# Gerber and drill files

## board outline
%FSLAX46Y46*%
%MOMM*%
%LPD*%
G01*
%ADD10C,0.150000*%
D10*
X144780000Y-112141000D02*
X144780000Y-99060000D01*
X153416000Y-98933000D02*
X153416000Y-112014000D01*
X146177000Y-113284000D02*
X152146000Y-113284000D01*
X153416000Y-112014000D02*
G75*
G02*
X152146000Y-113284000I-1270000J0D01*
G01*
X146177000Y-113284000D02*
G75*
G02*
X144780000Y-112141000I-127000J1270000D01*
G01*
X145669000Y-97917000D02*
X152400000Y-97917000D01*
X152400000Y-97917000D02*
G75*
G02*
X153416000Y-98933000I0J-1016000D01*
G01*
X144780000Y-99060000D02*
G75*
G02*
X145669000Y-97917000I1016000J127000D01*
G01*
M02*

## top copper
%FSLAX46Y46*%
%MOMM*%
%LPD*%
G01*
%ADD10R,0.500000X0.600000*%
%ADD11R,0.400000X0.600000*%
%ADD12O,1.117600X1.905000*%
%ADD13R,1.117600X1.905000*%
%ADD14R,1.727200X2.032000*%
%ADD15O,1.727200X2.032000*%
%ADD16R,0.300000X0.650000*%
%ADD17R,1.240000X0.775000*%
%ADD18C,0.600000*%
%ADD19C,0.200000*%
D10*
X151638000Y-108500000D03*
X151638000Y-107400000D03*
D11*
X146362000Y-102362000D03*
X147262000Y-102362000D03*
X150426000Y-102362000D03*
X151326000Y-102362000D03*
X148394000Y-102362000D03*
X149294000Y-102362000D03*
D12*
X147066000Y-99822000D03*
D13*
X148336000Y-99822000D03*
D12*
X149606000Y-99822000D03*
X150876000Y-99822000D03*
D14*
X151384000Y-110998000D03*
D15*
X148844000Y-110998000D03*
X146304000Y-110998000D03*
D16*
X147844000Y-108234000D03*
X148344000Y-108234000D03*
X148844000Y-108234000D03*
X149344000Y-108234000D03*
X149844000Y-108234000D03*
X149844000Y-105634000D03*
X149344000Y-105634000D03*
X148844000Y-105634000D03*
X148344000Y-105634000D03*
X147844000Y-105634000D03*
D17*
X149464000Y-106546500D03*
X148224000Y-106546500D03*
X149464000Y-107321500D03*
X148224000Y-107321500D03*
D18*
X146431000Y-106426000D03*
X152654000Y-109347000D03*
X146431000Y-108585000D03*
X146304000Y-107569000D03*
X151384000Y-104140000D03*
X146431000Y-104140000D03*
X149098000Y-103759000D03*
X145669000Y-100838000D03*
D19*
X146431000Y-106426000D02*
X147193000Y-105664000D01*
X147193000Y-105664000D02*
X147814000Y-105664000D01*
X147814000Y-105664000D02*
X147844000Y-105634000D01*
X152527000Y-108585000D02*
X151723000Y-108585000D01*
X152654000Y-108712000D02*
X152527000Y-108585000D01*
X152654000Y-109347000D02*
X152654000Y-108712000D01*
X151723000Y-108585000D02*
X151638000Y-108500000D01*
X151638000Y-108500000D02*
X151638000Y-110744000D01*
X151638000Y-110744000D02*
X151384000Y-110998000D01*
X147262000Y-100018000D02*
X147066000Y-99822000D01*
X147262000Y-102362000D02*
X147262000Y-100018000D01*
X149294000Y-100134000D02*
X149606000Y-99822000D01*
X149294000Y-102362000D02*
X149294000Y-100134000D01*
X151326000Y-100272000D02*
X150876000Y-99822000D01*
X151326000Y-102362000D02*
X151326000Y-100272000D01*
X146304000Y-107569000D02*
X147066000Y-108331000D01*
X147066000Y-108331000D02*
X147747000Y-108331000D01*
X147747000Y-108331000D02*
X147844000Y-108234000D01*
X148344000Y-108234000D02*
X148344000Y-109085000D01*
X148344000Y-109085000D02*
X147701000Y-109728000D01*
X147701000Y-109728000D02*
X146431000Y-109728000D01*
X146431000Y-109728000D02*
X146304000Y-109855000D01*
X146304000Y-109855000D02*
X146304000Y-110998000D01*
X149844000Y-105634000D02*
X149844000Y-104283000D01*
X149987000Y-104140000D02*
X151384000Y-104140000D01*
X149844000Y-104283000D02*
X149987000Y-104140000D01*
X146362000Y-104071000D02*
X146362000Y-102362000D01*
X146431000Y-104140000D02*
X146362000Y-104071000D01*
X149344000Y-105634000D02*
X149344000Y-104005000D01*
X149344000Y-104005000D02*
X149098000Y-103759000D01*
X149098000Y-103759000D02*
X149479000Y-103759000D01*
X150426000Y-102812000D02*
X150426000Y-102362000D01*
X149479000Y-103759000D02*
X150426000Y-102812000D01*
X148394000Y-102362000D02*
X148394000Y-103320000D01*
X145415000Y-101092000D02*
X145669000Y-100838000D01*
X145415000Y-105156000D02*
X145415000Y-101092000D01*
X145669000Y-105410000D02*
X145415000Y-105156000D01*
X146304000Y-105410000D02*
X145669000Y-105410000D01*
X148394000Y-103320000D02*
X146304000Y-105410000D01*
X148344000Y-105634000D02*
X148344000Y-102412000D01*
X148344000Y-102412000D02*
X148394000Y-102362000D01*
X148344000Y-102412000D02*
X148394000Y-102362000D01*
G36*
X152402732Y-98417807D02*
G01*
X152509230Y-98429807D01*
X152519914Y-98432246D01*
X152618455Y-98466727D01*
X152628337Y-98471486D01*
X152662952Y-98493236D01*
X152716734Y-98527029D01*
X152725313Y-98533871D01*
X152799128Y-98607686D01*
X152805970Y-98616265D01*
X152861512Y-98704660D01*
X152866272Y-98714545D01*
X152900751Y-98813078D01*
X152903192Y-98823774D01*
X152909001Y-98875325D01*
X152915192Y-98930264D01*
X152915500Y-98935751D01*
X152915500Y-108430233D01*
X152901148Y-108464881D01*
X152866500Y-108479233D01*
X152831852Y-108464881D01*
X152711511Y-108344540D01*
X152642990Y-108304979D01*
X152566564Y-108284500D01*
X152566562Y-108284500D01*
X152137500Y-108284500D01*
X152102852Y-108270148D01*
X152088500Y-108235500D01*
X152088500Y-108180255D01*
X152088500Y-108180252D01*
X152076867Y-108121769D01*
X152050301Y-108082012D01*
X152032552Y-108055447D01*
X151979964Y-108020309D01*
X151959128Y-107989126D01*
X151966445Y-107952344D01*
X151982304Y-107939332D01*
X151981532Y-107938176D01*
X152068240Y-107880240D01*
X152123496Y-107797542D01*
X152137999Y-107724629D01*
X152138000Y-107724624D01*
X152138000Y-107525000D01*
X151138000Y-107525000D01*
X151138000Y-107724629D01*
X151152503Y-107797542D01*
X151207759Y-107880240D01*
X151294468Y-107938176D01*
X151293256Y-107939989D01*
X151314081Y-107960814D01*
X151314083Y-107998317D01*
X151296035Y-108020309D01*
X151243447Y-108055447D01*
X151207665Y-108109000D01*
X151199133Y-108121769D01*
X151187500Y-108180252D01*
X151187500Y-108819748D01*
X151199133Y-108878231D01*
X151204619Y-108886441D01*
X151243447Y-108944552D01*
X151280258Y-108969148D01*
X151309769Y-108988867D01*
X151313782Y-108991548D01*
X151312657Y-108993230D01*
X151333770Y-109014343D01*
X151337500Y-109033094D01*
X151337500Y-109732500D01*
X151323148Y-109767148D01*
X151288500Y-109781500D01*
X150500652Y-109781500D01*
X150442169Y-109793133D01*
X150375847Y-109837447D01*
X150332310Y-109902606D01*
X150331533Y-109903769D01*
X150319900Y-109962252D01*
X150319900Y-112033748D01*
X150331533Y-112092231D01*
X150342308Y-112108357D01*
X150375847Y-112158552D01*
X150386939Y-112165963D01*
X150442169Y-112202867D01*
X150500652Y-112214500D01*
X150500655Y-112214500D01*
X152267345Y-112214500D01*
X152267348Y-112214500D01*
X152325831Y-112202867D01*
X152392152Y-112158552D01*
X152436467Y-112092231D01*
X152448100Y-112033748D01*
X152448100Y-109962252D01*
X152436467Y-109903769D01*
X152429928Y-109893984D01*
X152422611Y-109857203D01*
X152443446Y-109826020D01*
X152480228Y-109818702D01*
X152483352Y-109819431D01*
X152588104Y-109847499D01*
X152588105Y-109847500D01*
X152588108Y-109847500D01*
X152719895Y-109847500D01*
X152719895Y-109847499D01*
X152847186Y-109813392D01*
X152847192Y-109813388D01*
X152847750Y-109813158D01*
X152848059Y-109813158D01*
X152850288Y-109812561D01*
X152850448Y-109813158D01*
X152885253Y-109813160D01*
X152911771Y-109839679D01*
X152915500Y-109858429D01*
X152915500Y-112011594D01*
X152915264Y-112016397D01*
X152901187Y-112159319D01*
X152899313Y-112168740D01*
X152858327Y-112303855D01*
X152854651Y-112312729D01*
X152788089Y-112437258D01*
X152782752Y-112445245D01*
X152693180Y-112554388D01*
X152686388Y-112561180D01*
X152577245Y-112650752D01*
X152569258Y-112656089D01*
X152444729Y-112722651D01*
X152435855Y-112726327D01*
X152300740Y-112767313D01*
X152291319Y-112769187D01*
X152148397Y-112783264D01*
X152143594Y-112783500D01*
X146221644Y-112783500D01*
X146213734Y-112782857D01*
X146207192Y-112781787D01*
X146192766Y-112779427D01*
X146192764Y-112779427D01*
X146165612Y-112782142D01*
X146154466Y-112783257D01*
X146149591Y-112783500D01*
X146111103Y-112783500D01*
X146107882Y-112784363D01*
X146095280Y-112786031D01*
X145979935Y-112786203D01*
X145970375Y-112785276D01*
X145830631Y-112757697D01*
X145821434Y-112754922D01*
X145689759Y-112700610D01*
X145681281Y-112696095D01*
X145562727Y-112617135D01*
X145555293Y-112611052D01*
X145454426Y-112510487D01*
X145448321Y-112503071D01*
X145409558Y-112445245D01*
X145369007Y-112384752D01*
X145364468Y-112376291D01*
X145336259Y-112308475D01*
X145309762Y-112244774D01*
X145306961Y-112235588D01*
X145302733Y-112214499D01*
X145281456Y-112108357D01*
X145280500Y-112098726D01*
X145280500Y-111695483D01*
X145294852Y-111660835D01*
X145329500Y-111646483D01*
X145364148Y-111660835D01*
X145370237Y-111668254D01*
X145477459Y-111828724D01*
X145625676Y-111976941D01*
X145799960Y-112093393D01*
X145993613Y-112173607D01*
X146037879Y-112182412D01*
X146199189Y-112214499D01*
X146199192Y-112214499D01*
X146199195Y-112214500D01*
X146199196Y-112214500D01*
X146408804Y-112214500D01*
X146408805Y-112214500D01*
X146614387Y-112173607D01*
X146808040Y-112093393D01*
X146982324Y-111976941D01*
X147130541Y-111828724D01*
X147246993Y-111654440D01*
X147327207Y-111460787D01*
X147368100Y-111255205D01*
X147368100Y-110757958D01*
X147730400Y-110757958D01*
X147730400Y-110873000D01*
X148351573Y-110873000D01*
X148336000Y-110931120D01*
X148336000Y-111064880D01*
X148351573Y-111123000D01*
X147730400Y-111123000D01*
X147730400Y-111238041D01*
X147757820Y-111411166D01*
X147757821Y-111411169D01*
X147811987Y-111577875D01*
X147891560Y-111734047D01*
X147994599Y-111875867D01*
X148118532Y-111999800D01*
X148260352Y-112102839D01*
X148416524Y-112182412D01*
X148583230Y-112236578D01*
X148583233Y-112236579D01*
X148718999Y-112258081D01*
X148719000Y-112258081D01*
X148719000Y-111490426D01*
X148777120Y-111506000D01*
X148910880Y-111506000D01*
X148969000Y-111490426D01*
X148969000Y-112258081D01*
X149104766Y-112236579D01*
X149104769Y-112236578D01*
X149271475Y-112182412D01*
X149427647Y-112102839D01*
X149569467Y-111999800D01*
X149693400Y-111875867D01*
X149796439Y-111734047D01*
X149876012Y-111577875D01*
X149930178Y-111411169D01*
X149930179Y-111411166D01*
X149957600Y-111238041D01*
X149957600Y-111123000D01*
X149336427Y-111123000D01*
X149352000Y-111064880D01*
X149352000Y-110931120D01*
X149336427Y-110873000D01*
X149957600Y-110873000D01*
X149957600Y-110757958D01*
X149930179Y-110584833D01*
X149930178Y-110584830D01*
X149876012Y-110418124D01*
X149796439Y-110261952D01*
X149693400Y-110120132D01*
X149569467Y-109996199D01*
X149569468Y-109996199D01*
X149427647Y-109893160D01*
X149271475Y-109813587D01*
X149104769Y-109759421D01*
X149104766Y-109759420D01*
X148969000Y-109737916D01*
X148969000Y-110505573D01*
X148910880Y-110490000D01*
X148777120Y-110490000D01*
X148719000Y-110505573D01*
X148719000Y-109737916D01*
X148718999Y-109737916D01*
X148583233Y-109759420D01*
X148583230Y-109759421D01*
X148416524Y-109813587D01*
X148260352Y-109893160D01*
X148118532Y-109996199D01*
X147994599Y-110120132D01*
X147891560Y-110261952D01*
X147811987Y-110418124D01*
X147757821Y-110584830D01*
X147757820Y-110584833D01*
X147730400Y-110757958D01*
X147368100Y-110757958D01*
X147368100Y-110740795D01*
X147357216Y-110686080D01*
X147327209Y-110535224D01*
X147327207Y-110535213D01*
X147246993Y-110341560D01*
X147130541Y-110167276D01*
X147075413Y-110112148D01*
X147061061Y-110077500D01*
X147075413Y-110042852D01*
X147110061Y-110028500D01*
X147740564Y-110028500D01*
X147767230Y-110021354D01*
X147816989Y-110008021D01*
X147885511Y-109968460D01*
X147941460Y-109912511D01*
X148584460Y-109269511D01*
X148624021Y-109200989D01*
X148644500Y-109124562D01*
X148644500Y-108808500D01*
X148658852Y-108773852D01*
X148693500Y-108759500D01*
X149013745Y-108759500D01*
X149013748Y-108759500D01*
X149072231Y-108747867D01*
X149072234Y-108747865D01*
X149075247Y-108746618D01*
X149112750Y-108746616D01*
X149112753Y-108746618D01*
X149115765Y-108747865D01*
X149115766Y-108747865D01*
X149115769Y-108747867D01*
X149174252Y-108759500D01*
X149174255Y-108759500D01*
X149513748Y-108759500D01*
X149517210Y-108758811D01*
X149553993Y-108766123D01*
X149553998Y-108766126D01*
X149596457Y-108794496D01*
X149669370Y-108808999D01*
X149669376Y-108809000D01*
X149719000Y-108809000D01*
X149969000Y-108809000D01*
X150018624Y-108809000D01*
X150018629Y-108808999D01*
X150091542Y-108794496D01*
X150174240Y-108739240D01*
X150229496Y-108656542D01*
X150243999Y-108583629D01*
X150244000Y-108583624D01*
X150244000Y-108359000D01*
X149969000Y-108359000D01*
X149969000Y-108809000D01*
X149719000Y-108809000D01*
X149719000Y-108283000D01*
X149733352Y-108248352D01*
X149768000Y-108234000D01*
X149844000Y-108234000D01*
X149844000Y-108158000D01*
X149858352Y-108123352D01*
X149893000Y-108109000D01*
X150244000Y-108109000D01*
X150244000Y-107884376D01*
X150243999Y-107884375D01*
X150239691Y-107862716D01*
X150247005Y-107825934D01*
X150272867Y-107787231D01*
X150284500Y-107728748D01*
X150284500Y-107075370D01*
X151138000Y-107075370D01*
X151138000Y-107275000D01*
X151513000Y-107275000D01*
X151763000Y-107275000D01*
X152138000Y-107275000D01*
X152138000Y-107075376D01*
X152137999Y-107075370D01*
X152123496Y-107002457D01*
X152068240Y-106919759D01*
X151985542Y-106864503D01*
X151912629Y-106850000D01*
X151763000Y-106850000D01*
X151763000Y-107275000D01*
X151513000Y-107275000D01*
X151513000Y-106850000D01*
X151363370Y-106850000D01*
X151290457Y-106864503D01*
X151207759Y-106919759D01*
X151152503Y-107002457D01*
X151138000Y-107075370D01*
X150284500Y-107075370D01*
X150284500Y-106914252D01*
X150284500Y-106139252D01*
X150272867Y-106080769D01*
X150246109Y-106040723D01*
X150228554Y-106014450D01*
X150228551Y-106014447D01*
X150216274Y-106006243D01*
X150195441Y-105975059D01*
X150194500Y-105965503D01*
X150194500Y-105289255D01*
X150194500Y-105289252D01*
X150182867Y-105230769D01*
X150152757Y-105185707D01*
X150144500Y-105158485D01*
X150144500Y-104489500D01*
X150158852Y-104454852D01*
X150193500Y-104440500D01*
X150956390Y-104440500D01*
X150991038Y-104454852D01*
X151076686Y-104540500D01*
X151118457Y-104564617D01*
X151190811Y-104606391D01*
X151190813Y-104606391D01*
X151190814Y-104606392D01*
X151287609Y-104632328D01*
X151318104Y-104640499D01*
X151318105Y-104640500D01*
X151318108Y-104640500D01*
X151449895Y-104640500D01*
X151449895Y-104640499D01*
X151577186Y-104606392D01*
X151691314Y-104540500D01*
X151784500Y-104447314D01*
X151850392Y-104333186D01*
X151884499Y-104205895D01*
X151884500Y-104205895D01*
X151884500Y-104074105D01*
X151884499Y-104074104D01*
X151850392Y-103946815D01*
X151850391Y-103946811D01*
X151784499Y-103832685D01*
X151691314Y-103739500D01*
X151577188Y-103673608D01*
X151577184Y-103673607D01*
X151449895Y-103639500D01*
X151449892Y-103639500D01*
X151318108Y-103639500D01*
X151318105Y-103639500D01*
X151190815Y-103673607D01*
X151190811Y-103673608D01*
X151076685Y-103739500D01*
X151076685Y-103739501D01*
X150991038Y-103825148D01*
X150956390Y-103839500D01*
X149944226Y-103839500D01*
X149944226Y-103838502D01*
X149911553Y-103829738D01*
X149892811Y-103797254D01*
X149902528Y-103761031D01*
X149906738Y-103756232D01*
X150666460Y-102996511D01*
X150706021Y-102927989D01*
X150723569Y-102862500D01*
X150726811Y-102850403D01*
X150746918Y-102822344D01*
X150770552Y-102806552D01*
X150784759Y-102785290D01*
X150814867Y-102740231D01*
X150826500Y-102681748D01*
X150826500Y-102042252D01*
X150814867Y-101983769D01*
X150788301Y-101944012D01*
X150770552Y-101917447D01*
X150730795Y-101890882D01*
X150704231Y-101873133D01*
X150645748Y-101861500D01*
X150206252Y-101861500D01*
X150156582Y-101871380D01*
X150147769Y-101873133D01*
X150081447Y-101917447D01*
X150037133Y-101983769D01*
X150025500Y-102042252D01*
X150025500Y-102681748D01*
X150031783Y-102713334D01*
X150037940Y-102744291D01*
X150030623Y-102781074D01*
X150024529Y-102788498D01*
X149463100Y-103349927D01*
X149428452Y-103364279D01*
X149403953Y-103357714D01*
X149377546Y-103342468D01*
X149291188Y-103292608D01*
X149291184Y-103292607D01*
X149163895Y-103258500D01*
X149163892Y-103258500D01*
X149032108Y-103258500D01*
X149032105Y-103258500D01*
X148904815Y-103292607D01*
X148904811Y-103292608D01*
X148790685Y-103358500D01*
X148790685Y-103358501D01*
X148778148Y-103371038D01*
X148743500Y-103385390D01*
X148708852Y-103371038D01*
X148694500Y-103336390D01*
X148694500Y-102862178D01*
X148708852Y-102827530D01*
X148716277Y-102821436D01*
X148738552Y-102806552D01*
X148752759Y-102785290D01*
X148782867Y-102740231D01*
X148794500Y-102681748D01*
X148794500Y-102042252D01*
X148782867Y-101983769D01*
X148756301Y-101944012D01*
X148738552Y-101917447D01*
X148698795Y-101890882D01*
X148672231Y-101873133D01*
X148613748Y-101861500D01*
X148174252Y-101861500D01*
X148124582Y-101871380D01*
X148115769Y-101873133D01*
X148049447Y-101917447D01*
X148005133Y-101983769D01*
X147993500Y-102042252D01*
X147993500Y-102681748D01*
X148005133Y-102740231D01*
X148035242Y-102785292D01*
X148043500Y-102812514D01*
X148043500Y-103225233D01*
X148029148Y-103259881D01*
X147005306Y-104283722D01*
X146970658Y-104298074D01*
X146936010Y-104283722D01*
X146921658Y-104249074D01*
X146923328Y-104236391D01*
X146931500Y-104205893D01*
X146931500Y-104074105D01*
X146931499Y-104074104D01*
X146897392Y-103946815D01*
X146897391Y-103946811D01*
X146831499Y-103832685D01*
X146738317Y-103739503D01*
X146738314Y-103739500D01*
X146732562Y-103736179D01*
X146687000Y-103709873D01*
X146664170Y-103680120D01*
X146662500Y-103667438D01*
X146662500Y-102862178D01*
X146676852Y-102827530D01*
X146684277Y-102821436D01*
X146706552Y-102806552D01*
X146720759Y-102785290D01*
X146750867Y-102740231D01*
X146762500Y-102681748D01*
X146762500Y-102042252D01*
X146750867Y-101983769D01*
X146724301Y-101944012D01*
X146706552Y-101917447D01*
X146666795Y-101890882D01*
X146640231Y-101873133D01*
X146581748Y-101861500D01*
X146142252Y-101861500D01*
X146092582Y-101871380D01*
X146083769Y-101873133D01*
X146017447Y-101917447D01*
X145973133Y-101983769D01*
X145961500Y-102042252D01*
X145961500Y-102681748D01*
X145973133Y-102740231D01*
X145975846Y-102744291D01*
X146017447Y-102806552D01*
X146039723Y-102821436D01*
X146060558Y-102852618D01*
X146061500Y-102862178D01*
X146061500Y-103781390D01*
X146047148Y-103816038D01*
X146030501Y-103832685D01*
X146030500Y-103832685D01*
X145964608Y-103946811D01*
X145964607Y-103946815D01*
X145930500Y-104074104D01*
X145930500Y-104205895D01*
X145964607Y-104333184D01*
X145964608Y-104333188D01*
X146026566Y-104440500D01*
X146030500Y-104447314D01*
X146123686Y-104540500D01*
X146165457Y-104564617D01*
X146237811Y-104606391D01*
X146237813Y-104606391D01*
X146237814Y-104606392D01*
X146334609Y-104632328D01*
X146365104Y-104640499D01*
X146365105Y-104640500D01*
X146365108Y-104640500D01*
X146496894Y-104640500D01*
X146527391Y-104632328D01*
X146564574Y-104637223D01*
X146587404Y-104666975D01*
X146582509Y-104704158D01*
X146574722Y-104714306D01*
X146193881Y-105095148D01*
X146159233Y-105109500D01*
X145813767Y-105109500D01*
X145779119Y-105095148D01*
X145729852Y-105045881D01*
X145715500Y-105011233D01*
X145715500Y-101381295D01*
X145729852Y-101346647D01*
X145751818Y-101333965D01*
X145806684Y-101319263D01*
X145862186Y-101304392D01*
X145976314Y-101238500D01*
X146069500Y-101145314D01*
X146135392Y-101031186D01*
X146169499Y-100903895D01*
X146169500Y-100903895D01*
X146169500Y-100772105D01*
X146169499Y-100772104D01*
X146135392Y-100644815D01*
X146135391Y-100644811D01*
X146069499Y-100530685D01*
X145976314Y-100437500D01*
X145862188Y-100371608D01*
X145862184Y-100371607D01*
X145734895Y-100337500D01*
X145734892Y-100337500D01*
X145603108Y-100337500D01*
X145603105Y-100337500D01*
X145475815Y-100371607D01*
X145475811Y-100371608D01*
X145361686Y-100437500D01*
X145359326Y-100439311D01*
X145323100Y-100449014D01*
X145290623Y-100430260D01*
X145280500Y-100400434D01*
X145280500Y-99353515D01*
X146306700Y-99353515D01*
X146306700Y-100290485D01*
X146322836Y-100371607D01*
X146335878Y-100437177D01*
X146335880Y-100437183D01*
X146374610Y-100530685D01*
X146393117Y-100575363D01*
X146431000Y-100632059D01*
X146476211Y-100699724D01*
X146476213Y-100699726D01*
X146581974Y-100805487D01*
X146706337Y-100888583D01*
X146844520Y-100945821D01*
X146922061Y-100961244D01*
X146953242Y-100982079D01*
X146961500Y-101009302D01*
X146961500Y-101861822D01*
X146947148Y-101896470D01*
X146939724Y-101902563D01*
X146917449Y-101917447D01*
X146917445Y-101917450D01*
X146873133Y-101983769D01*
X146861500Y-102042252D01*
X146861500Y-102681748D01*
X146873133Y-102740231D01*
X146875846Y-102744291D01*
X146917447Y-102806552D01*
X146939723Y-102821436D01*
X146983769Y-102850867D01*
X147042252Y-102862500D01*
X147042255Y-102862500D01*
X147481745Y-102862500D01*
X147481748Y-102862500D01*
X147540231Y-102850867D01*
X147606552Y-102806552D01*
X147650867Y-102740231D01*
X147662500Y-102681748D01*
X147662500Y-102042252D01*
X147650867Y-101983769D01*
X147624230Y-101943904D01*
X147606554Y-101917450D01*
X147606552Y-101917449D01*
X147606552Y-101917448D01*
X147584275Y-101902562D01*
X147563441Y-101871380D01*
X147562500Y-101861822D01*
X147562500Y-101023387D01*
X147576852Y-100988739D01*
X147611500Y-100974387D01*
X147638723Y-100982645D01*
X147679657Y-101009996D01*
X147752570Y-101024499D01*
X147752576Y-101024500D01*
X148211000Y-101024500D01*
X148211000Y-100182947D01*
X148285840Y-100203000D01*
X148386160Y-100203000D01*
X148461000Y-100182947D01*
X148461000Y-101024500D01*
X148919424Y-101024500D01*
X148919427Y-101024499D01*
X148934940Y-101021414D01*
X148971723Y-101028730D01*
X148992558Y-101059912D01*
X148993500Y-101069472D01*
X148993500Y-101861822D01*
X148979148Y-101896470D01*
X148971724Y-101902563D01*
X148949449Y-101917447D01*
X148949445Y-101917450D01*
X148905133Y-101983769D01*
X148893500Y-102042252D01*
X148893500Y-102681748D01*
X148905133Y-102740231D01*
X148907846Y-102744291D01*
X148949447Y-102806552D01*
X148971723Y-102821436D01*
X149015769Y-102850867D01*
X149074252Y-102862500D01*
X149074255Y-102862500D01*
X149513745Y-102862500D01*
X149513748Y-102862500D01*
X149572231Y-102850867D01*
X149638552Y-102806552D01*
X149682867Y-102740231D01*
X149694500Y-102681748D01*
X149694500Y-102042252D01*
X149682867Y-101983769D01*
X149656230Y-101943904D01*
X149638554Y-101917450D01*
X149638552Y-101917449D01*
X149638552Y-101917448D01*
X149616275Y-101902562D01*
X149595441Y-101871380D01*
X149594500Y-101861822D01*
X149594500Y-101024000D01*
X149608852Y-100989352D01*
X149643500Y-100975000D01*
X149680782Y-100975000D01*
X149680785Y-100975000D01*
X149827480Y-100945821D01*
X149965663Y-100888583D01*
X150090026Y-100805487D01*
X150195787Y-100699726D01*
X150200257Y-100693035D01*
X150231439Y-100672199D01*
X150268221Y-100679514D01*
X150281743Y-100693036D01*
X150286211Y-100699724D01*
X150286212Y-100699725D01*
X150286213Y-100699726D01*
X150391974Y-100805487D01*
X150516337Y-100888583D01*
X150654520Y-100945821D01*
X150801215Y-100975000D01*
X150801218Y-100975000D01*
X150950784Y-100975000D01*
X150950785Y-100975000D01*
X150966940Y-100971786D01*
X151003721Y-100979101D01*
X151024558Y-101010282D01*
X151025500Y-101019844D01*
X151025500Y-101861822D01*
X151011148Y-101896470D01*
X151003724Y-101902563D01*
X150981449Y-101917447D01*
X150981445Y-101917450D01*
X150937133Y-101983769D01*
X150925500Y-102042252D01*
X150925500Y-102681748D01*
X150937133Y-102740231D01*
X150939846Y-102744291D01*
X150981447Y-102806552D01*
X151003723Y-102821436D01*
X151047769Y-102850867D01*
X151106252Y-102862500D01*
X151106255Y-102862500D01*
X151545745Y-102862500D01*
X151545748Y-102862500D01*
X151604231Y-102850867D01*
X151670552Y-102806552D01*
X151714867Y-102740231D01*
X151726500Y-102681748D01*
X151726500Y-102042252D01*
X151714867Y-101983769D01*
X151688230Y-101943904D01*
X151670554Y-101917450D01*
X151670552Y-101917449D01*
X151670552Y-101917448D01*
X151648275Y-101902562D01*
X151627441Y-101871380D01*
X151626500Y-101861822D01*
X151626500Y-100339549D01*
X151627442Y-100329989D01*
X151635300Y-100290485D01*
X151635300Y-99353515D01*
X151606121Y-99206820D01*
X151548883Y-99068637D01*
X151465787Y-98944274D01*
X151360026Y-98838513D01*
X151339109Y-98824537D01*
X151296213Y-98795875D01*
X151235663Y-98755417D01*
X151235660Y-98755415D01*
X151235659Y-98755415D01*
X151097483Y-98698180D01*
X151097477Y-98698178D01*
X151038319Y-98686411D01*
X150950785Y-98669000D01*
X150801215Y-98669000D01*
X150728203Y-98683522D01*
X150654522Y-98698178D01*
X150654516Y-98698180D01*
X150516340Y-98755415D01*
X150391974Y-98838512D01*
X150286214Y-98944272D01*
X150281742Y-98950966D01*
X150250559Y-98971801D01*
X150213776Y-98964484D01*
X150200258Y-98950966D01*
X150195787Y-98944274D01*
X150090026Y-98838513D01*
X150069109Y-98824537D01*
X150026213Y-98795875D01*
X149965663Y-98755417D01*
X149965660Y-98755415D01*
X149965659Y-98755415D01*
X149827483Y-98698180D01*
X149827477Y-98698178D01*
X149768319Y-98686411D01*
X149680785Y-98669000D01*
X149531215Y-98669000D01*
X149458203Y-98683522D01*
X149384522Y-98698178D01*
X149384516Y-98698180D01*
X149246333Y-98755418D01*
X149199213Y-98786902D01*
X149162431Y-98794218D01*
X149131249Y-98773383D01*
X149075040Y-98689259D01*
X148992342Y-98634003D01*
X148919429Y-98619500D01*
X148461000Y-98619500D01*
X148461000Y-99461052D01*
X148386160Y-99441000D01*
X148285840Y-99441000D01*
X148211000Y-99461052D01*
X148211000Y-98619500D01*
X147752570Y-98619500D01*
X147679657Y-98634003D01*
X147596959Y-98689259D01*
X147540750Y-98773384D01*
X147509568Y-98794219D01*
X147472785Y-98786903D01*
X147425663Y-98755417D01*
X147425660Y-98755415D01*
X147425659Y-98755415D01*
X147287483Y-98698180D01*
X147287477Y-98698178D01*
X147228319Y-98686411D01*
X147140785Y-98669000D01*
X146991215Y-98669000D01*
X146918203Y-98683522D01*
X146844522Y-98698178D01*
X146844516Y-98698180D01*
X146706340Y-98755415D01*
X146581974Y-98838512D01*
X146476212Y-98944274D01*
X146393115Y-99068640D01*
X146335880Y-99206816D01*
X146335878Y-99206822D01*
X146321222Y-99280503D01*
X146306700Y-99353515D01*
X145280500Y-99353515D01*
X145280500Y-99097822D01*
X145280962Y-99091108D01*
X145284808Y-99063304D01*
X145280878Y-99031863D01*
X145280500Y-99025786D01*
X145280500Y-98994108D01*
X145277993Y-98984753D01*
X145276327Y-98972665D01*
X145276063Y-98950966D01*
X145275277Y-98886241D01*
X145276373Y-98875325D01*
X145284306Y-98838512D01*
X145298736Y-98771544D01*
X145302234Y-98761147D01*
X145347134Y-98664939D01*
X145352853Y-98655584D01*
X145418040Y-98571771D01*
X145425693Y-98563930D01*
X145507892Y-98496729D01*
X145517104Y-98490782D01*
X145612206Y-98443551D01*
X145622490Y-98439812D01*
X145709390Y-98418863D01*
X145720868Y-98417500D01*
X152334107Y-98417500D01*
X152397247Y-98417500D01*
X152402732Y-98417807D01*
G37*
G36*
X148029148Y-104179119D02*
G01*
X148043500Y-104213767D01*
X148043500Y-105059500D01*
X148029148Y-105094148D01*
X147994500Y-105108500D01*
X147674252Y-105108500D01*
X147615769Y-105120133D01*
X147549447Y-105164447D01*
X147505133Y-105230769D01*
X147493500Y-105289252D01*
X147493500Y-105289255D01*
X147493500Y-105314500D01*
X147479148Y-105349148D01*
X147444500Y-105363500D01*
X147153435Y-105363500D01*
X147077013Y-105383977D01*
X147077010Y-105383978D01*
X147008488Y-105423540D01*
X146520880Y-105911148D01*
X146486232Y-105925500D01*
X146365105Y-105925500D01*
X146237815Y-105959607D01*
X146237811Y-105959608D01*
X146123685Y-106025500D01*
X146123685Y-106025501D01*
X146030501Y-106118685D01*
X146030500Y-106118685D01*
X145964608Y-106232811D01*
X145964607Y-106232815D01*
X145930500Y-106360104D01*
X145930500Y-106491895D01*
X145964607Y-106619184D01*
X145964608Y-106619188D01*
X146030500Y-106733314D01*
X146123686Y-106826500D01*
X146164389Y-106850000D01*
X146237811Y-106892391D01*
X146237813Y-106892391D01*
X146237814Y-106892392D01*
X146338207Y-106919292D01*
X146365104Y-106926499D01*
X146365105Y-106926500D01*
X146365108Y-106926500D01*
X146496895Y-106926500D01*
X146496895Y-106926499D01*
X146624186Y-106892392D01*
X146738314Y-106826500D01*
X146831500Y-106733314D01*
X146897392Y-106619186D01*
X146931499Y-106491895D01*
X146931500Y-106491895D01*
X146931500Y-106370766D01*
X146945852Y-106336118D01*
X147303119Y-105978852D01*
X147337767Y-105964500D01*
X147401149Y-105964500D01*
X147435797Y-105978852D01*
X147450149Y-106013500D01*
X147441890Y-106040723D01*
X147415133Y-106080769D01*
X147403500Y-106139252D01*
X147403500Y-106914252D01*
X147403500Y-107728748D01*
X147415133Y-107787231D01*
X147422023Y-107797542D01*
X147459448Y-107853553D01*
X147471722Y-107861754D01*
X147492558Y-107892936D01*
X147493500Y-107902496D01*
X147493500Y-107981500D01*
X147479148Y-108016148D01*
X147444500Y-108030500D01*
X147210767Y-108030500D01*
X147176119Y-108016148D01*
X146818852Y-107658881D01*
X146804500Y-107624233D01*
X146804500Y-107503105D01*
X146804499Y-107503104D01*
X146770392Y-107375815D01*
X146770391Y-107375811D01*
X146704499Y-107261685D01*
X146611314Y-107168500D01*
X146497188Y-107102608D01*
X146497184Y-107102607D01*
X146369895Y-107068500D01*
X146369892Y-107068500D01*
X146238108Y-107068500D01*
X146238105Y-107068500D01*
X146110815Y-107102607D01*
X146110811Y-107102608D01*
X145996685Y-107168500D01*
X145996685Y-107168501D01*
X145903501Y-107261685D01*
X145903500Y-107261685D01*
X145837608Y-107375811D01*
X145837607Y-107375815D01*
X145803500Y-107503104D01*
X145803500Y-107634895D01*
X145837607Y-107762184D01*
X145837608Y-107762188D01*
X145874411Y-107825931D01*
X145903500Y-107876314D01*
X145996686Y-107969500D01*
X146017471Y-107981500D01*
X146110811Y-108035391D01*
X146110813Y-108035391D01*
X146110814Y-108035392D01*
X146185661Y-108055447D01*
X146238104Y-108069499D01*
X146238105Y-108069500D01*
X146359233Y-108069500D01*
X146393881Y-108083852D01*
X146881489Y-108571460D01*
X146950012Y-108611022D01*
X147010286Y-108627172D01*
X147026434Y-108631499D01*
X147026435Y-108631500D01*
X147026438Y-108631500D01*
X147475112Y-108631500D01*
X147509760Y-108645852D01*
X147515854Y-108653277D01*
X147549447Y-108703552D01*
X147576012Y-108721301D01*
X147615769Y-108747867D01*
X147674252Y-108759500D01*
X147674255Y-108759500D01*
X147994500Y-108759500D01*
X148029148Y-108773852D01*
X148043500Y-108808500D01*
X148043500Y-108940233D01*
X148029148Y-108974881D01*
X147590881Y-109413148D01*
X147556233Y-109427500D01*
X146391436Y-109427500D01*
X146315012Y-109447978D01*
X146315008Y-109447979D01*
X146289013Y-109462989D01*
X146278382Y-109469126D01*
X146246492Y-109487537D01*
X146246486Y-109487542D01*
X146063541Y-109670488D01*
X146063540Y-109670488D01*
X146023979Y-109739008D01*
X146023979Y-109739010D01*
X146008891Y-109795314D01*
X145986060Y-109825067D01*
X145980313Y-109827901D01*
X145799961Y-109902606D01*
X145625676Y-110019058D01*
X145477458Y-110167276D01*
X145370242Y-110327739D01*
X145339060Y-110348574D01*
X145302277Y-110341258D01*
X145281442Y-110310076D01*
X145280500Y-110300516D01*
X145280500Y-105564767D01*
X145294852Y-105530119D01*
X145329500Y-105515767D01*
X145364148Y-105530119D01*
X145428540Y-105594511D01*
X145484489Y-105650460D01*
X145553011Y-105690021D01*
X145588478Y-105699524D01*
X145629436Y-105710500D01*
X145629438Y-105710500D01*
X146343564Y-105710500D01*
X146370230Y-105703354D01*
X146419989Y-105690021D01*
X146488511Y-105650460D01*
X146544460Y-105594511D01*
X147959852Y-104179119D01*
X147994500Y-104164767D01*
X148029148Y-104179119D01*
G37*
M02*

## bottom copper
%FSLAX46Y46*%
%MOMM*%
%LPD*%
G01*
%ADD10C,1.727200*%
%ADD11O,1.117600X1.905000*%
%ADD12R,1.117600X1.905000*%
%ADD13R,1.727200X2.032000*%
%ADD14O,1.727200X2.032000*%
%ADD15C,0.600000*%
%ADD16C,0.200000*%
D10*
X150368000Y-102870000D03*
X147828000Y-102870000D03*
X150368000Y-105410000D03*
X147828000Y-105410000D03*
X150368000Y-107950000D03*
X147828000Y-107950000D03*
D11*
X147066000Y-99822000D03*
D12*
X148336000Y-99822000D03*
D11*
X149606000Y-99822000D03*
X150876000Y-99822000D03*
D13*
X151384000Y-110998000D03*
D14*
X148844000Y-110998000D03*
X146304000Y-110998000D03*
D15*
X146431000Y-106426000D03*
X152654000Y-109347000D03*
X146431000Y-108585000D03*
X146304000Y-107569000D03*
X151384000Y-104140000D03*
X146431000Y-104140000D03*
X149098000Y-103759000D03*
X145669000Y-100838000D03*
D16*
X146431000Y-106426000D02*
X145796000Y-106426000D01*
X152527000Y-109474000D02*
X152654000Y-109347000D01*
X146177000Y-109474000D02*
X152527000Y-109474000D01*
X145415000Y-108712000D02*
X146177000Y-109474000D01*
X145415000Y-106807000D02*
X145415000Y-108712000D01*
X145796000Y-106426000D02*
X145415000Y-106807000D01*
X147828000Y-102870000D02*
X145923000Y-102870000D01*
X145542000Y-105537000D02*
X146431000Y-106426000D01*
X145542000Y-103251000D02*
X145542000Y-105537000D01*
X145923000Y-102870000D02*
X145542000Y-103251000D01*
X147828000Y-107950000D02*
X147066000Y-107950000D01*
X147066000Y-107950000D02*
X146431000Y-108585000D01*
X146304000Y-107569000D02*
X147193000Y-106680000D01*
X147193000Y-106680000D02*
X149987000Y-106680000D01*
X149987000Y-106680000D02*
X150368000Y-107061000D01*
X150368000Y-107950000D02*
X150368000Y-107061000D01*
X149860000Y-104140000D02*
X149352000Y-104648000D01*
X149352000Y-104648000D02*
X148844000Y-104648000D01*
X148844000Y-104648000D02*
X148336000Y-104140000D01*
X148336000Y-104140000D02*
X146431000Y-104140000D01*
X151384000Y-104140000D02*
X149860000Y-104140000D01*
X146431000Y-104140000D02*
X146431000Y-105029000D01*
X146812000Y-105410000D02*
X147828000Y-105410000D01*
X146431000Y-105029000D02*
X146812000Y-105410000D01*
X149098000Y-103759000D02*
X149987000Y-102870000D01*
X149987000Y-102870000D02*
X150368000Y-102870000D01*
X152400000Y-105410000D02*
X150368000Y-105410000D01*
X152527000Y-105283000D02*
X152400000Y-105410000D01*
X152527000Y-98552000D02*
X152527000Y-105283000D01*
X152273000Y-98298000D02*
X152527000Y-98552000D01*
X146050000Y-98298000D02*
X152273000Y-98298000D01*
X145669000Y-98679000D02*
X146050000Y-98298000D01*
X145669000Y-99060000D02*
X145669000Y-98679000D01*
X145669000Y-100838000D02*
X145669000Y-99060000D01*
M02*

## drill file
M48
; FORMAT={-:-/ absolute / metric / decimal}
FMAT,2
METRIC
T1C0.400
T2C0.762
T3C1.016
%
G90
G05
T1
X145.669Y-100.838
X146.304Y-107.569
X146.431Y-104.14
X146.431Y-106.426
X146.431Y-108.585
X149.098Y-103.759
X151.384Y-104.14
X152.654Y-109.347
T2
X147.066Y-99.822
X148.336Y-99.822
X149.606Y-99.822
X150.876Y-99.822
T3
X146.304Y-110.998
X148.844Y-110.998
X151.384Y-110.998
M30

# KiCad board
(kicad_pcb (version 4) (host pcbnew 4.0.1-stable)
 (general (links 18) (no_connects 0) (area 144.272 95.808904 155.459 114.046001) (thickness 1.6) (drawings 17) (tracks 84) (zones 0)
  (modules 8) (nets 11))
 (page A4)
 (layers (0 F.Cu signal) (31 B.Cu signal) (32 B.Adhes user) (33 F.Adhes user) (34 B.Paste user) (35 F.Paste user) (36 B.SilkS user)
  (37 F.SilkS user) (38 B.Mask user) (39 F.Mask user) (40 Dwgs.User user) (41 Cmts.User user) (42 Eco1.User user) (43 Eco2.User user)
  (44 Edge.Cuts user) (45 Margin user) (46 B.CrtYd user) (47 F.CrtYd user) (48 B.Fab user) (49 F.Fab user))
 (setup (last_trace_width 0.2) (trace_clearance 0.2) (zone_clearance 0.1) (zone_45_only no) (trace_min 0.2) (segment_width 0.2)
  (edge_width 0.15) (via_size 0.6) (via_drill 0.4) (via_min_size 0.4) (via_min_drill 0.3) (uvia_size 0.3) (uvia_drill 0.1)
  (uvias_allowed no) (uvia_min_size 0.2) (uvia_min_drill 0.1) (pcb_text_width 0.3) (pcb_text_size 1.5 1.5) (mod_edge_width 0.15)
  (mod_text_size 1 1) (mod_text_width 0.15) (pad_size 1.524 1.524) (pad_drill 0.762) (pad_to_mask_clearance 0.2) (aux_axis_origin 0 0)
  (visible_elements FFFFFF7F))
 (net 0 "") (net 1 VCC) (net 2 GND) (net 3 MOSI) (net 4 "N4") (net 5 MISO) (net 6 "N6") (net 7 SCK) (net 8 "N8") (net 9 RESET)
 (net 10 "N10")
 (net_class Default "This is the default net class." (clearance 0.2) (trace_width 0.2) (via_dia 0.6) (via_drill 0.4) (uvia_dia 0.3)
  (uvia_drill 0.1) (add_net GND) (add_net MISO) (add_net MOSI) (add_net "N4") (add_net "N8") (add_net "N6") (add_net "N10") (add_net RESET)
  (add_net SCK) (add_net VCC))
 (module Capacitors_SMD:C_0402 (layer F.Cu) (at 151.638 107.95 90)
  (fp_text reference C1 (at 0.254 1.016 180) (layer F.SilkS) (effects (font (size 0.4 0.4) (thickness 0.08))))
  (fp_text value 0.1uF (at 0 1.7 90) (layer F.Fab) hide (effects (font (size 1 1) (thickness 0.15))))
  (pad 1 smd rect (at -0.55 0 90) (size 0.6 0.5) (layers F.Cu F.Paste F.Mask) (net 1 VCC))
  (pad 2 smd rect (at 0.55 0 90) (size 0.6 0.5) (layers F.Cu F.Paste F.Mask) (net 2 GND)))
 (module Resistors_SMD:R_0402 (layer F.Cu) (at 146.812 102.362)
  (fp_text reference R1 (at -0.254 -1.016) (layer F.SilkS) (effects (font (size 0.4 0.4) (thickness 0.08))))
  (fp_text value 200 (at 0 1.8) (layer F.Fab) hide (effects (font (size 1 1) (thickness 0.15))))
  (pad 1 smd rect (at -0.45 0) (size 0.4 0.6) (layers F.Cu F.Paste F.Mask) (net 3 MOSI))
  (pad 2 smd rect (at 0.45 0) (size 0.4 0.6) (layers F.Cu F.Paste F.Mask) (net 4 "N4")))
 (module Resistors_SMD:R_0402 (layer F.Cu) (at 150.876 102.362)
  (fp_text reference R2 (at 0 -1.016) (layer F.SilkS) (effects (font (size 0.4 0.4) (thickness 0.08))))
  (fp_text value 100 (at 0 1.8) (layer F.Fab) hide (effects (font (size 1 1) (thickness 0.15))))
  (pad 1 smd rect (at -0.45 0) (size 0.4 0.6) (layers F.Cu F.Paste F.Mask) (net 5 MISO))
  (pad 2 smd rect (at 0.45 0) (size 0.4 0.6) (layers F.Cu F.Paste F.Mask) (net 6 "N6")))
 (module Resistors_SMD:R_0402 (layer F.Cu) (at 148.844 102.362)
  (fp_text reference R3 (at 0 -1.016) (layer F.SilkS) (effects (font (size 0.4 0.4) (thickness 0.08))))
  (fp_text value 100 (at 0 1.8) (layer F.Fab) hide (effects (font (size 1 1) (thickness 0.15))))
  (pad 1 smd rect (at -0.45 0) (size 0.4 0.6) (layers F.Cu F.Paste F.Mask) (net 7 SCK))
  (pad 2 smd rect (at 0.45 0) (size 0.4 0.6) (layers F.Cu F.Paste F.Mask) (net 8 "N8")))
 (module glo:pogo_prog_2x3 (layer B.Cu) (at 150.368 102.87 180)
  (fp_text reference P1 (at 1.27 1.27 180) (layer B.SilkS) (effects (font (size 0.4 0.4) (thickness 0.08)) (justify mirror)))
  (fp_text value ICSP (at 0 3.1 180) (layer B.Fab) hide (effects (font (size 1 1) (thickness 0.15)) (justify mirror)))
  (pad 1 smd circle (at 0 0 180) (size 1.7272 1.7272) (layers B.Cu B.Paste B.Mask) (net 5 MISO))
  (pad 2 smd circle (at 2.54 0 180) (size 1.7272 1.7272) (layers B.Cu B.Paste B.Mask) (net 1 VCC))
  (pad 3 smd circle (at 0 -2.54 180) (size 1.7272 1.7272) (layers B.Cu B.Paste B.Mask) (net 7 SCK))
  (pad 4 smd circle (at 2.54 -2.54 180) (size 1.7272 1.7272) (layers B.Cu B.Paste B.Mask) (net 3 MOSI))
  (pad 5 smd circle (at 0 -5.08 180) (size 1.7272 1.7272) (layers B.Cu B.Paste B.Mask) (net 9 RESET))
  (pad 6 smd circle (at 2.54 -5.08 180) (size 1.7272 1.7272) (layers B.Cu B.Paste B.Mask) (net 2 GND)))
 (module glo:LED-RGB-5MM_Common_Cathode (layer F.Cu) (at 147.066 99.822 90)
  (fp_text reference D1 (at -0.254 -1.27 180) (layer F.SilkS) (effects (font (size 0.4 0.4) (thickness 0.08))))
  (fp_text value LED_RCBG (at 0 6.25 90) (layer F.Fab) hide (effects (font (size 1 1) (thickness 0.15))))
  (pad 1 thru_hole oval (at 0 0 90) (size 1.905 1.1176) (drill 0.762) (layers *.Cu *.Mask F.SilkS) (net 4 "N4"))
  (pad 2 thru_hole rect (at 0 1.27 90) (size 1.905 1.1176) (drill 0.762) (layers *.Cu *.Mask F.SilkS) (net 2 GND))
  (pad 3 thru_hole oval (at 0 2.54 90) (size 1.905 1.1176) (drill 0.762) (layers *.Cu *.Mask F.SilkS) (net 8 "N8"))
  (pad 4 thru_hole oval (at 0 3.81 90) (size 1.905 1.1176) (drill 0.762) (layers *.Cu *.Mask F.SilkS) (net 6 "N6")))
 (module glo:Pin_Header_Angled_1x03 (layer F.Cu) (at 151.384 110.998 270)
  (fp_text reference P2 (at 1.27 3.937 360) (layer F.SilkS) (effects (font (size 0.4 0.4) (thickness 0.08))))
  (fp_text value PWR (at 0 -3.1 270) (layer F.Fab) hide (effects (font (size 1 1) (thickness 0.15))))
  (pad 1 thru_hole rect (at 0 0 270) (size 2.032 1.7272) (drill 1.016) (layers *.Cu *.Mask F.SilkS) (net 1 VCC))
  (pad 2 thru_hole oval (at 0 2.54 270) (size 2.032 1.7272) (drill 1.016) (layers *.Cu *.Mask F.SilkS) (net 2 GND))
  (pad 3 thru_hole oval (at 0 5.08 270) (size 2.032 1.7272) (drill 1.016) (layers *.Cu *.Mask F.SilkS) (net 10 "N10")))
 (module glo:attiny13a (layer F.Cu) (at 148.844 106.934 90)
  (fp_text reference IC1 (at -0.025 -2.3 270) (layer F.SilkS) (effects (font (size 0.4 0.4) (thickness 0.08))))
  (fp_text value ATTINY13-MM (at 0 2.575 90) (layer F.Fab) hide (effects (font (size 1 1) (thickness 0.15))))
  (pad 1 smd rect (at -1.3 -1 90) (size 0.65 0.3) (layers F.Cu F.Paste F.Mask) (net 9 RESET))
  (pad 2 smd rect (at -1.3 -0.5 90) (size 0.65 0.3) (layers F.Cu F.Paste F.Mask) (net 10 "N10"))
  (pad 3 smd rect (at -1.3 0 90) (size 0.65 0.3) (layers F.Cu F.Paste F.Mask))
  (pad 4 smd rect (at -1.3 0.5 90) (size 0.65 0.3) (layers F.Cu F.Paste F.Mask))
  (pad 5 smd rect (at -1.3 1 90) (size 0.65 0.3) (layers F.Cu F.Paste F.Mask) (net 2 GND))
  (pad 6 smd rect (at 1.3 1 90) (size 0.65 0.3) (layers F.Cu F.Paste F.Mask) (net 3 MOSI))
  (pad 7 smd rect (at 1.3 0.5 90) (size 0.65 0.3) (layers F.Cu F.Paste F.Mask) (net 5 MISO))
  (pad 8 smd rect (at 1.3 0 90) (size 0.65 0.3) (layers F.Cu F.Paste F.Mask))
  (pad 9 smd rect (at 1.3 -0.5 90) (size 0.65 0.3) (layers F.Cu F.Paste F.Mask) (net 7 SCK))
  (pad 10 smd rect (at 1.3 -1 90) (size 0.65 0.3) (layers F.Cu F.Paste F.Mask) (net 1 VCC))
  (pad "" smd rect (at 0.3875 0.62 90) (size 0.775 1.24) (layers F.Cu F.Paste F.Mask) (solder_paste_margin_ratio -0.2))
  (pad "" smd rect (at 0.3875 -0.62 90) (size 0.775 1.24) (layers F.Cu F.Paste F.Mask) (solder_paste_margin_ratio -0.2))
  (pad "" smd rect (at -0.3875 0.62 90) (size 0.775 1.24) (layers F.Cu F.Paste F.Mask) (solder_paste_margin_ratio -0.2))
  (pad "" smd rect (at -0.3875 -0.62 90) (size 0.775 1.24) (layers F.Cu F.Paste F.Mask) (solder_paste_margin_ratio -0.2)))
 (gr_line (start 144.78 112.141) (end 144.78 99.06) (angle 90) (layer Edge.Cuts) (width 0.15))
 (gr_line (start 153.416 98.933) (end 153.416 112.014) (angle 90) (layer Edge.Cuts) (width 0.15))
 (gr_line (start 146.177 113.284) (end 152.146 113.284) (angle 90) (layer Edge.Cuts) (width 0.15))
 (gr_arc (start 152.146 112.014) (end 153.416 112.014) (angle 90) (layer Edge.Cuts) (width 0.15))
 (gr_arc (start 146.05 112.014) (end 146.177 113.284) (angle 90) (layer Edge.Cuts) (width 0.15))
 (gr_line (start 145.669 97.917) (end 152.4 97.917) (angle 90) (layer Edge.Cuts) (width 0.15))
 (gr_arc (start 152.4 98.933) (end 152.4 97.917) (angle 90) (layer Edge.Cuts) (width 0.15))
 (gr_arc (start 145.796 98.933) (end 144.78 99.06) (angle 90) (layer Edge.Cuts) (width 0.15))
 (segment (start 146.431 106.426) (end 147.193 105.664) (width 0.2) (layer F.Cu) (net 1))
 (via (at 146.431 106.426) (size 0.6) (drill 0.4) (layers F.Cu B.Cu) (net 1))
 (segment (start 147.193 105.664) (end 147.814 105.664) (width 0.2) (layer F.Cu) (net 1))
 (segment (start 147.814 105.664) (end 147.844 105.634) (width 0.2) (layer F.Cu) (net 1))
 (segment (start 146.431 106.426) (end 145.796 106.426) (width 0.2) (layer B.Cu) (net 1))
 (segment (start 152.527 108.585) (end 151.723 108.585) (width 0.2) (layer F.Cu) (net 1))
 (segment (start 152.654 108.712) (end 152.527 108.585) (width 0.2) (layer F.Cu) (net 1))
 (segment (start 152.654 109.347) (end 152.654 108.712) (width 0.2) (layer F.Cu) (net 1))
 (via (at 152.654 109.347) (size 0.6) (drill 0.4) (layers F.Cu B.Cu) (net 1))
 (segment (start 152.527 109.474) (end 152.654 109.347) (width 0.2) (layer B.Cu) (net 1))
 (segment (start 146.177 109.474) (end 152.527 109.474) (width 0.2) (layer B.Cu) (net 1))
 (segment (start 145.415 108.712) (end 146.177 109.474) (width 0.2) (layer B.Cu) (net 1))
 (segment (start 145.415 106.807) (end 145.415 108.712) (width 0.2) (layer B.Cu) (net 1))
 (segment (start 145.796 106.426) (end 145.415 106.807) (width 0.2) (layer B.Cu) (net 1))
 (segment (start 151.723 108.585) (end 151.638 108.5) (width 0.2) (layer F.Cu) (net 1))
 (segment (start 147.828 102.87) (end 145.923 102.87) (width 0.2) (layer B.Cu) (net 1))
 (segment (start 145.542 105.537) (end 146.431 106.426) (width 0.2) (layer B.Cu) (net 1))
 (segment (start 145.542 103.251) (end 145.542 105.537) (width 0.2) (layer B.Cu) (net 1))
 (segment (start 145.923 102.87) (end 145.542 103.251) (width 0.2) (layer B.Cu) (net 1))
 (segment (start 151.638 108.5) (end 151.638 110.744) (width 0.2) (layer F.Cu) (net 1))
 (segment (start 151.638 110.744) (end 151.384 110.998) (width 0.2) (layer F.Cu) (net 1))
 (segment (start 147.828 107.95) (end 147.066 107.95) (width 0.2) (layer B.Cu) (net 2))
 (segment (start 147.066 107.95) (end 146.431 108.585) (width 0.2) (layer B.Cu) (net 2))
 (via (at 146.431 108.585) (size 0.6) (drill 0.4) (layers F.Cu B.Cu) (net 2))
 (segment (start 147.262 100.018) (end 147.066 99.822) (width 0.2) (layer F.Cu) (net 4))
 (segment (start 147.262 102.362) (end 147.262 100.018) (width 0.2) (layer F.Cu) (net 4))
 (segment (start 149.294 100.134) (end 149.606 99.822) (width 0.2) (layer F.Cu) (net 8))
 (segment (start 149.294 102.362) (end 149.294 100.134) (width 0.2) (layer F.Cu) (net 8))
 (segment (start 151.326 100.272) (end 150.876 99.822) (width 0.2) (layer F.Cu) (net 6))
 (segment (start 151.326 102.362) (end 151.326 100.272) (width 0.2) (layer F.Cu) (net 6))
 (segment (start 146.304 107.569) (end 147.066 108.331) (width 0.2) (layer F.Cu) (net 9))
 (via (at 146.304 107.569) (size 0.6) (drill 0.4) (layers F.Cu B.Cu) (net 9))
 (segment (start 146.304 107.569) (end 147.193 106.68) (width 0.2) (layer B.Cu) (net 9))
 (segment (start 147.193 106.68) (end 149.987 106.68) (width 0.2) (layer B.Cu) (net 9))
 (segment (start 149.987 106.68) (end 150.368 107.061) (width 0.2) (layer B.Cu) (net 9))
 (segment (start 150.368 107.95) (end 150.368 107.061) (width 0.2) (layer B.Cu) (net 9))
 (segment (start 147.066 108.331) (end 147.747 108.331) (width 0.2) (layer F.Cu) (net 9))
 (segment (start 147.747 108.331) (end 147.844 108.234) (width 0.2) (layer F.Cu) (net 9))
 (segment (start 148.344 108.234) (end 148.344 109.085) (width 0.2) (layer F.Cu) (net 10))
 (segment (start 148.344 109.085) (end 147.701 109.728) (width 0.2) (layer F.Cu) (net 10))
 (segment (start 147.701 109.728) (end 146.431 109.728) (width 0.2) (layer F.Cu) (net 10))
 (segment (start 146.431 109.728) (end 146.304 109.855) (width 0.2) (layer F.Cu) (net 10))
 (segment (start 146.304 109.855) (end 146.304 110.998) (width 0.2) (layer F.Cu) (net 10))
 (segment (start 149.844 105.634) (end 149.844 104.283) (width 0.2) (layer F.Cu) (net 3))
 (segment (start 149.86 104.14) (end 149.352 104.648) (width 0.2) (layer B.Cu) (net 3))
 (segment (start 149.352 104.648) (end 148.844 104.648) (width 0.2) (layer B.Cu) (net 3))
 (segment (start 148.844 104.648) (end 148.336 104.14) (width 0.2) (layer B.Cu) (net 3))
 (segment (start 148.336 104.14) (end 146.431 104.14) (width 0.2) (layer B.Cu) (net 3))
 (via (at 151.384 104.14) (size 0.6) (drill 0.4) (layers F.Cu B.Cu) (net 3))
 (segment (start 149.987 104.14) (end 151.384 104.14) (width 0.2) (layer F.Cu) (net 3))
 (segment (start 149.844 104.283) (end 149.987 104.14) (width 0.2) (layer F.Cu) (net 3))
 (segment (start 151.384 104.14) (end 149.86 104.14) (width 0.2) (layer B.Cu) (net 3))
 (segment (start 146.431 104.14) (end 146.431 105.029) (width 0.2) (layer B.Cu) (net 3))
 (segment (start 146.812 105.41) (end 147.828 105.41) (width 0.2) (layer B.Cu) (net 3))
 (segment (start 146.431 105.029) (end 146.812 105.41) (width 0.2) (layer B.Cu) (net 3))
 (segment (start 146.362 104.071) (end 146.362 102.362) (width 0.2) (layer F.Cu) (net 3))
 (segment (start 146.431 104.14) (end 146.362 104.071) (width 0.2) (layer F.Cu) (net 3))
 (via (at 146.431 104.14) (size 0.6) (drill 0.4) (layers F.Cu B.Cu) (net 3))
 (segment (start 149.344 105.634) (end 149.344 104.005) (width 0.2) (layer F.Cu) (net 5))
 (segment (start 149.344 104.005) (end 149.098 103.759) (width 0.2) (layer F.Cu) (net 5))
 (segment (start 149.098 103.759) (end 149.479 103.759) (width 0.2) (layer F.Cu) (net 5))
 (segment (start 150.426 102.812) (end 150.426 102.362) (width 0.2) (layer F.Cu) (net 5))
 (segment (start 149.479 103.759) (end 150.426 102.812) (width 0.2) (layer F.Cu) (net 5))
 (segment (start 149.098 103.759) (end 149.987 102.87) (width 0.2) (layer B.Cu) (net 5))
 (via (at 149.098 103.759) (size 0.6) (drill 0.4) (layers F.Cu B.Cu) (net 5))
 (segment (start 149.987 102.87) (end 150.368 102.87) (width 0.2) (layer B.Cu) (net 5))
 (segment (start 148.394 102.362) (end 148.394 103.32) (width 0.2) (layer F.Cu) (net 7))
 (segment (start 152.4 105.41) (end 150.368 105.41) (width 0.2) (layer B.Cu) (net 7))
 (segment (start 152.527 105.283) (end 152.4 105.41) (width 0.2) (layer B.Cu) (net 7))
 (segment (start 152.527 98.552) (end 152.527 105.283) (width 0.2) (layer B.Cu) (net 7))
 (segment (start 152.273 98.298) (end 152.527 98.552) (width 0.2) (layer B.Cu) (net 7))
 (segment (start 146.05 98.298) (end 152.273 98.298) (width 0.2) (layer B.Cu) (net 7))
 (segment (start 145.669 98.679) (end 146.05 98.298) (width 0.2) (layer B.Cu) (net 7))
 (segment (start 145.669 99.06) (end 145.669 98.679) (width 0.2) (layer B.Cu) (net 7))
 (segment (start 145.669 100.838) (end 145.669 99.06) (width 0.2) (layer B.Cu) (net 7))
 (via (at 145.669 100.838) (size 0.6) (drill 0.4) (layers F.Cu B.Cu) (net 7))
 (segment (start 145.415 101.092) (end 145.669 100.838) (width 0.2) (layer F.Cu) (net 7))
 (segment (start 145.415 105.156) (end 145.415 101.092) (width 0.2) (layer F.Cu) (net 7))
 (segment (start 145.669 105.41) (end 145.415 105.156) (width 0.2) (layer F.Cu) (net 7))
 (segment (start 146.304 105.41) (end 145.669 105.41) (width 0.2) (layer F.Cu) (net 7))
 (segment (start 148.394 103.32) (end 146.304 105.41) (width 0.2) (layer F.Cu) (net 7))
 (segment (start 148.344 105.634) (end 148.344 102.412) (width 0.2) (layer F.Cu) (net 7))
 (segment (start 148.344 102.412) (end 148.394 102.362) (width 0.2) (layer F.Cu) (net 7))
 (segment (start 148.344 102.412) (end 148.394 102.362) (width 0.2) (layer F.Cu) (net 7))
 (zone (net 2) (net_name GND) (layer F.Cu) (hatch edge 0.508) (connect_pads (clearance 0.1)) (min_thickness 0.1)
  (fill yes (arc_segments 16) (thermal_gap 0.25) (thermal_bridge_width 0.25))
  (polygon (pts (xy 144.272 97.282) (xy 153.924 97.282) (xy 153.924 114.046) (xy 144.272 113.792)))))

